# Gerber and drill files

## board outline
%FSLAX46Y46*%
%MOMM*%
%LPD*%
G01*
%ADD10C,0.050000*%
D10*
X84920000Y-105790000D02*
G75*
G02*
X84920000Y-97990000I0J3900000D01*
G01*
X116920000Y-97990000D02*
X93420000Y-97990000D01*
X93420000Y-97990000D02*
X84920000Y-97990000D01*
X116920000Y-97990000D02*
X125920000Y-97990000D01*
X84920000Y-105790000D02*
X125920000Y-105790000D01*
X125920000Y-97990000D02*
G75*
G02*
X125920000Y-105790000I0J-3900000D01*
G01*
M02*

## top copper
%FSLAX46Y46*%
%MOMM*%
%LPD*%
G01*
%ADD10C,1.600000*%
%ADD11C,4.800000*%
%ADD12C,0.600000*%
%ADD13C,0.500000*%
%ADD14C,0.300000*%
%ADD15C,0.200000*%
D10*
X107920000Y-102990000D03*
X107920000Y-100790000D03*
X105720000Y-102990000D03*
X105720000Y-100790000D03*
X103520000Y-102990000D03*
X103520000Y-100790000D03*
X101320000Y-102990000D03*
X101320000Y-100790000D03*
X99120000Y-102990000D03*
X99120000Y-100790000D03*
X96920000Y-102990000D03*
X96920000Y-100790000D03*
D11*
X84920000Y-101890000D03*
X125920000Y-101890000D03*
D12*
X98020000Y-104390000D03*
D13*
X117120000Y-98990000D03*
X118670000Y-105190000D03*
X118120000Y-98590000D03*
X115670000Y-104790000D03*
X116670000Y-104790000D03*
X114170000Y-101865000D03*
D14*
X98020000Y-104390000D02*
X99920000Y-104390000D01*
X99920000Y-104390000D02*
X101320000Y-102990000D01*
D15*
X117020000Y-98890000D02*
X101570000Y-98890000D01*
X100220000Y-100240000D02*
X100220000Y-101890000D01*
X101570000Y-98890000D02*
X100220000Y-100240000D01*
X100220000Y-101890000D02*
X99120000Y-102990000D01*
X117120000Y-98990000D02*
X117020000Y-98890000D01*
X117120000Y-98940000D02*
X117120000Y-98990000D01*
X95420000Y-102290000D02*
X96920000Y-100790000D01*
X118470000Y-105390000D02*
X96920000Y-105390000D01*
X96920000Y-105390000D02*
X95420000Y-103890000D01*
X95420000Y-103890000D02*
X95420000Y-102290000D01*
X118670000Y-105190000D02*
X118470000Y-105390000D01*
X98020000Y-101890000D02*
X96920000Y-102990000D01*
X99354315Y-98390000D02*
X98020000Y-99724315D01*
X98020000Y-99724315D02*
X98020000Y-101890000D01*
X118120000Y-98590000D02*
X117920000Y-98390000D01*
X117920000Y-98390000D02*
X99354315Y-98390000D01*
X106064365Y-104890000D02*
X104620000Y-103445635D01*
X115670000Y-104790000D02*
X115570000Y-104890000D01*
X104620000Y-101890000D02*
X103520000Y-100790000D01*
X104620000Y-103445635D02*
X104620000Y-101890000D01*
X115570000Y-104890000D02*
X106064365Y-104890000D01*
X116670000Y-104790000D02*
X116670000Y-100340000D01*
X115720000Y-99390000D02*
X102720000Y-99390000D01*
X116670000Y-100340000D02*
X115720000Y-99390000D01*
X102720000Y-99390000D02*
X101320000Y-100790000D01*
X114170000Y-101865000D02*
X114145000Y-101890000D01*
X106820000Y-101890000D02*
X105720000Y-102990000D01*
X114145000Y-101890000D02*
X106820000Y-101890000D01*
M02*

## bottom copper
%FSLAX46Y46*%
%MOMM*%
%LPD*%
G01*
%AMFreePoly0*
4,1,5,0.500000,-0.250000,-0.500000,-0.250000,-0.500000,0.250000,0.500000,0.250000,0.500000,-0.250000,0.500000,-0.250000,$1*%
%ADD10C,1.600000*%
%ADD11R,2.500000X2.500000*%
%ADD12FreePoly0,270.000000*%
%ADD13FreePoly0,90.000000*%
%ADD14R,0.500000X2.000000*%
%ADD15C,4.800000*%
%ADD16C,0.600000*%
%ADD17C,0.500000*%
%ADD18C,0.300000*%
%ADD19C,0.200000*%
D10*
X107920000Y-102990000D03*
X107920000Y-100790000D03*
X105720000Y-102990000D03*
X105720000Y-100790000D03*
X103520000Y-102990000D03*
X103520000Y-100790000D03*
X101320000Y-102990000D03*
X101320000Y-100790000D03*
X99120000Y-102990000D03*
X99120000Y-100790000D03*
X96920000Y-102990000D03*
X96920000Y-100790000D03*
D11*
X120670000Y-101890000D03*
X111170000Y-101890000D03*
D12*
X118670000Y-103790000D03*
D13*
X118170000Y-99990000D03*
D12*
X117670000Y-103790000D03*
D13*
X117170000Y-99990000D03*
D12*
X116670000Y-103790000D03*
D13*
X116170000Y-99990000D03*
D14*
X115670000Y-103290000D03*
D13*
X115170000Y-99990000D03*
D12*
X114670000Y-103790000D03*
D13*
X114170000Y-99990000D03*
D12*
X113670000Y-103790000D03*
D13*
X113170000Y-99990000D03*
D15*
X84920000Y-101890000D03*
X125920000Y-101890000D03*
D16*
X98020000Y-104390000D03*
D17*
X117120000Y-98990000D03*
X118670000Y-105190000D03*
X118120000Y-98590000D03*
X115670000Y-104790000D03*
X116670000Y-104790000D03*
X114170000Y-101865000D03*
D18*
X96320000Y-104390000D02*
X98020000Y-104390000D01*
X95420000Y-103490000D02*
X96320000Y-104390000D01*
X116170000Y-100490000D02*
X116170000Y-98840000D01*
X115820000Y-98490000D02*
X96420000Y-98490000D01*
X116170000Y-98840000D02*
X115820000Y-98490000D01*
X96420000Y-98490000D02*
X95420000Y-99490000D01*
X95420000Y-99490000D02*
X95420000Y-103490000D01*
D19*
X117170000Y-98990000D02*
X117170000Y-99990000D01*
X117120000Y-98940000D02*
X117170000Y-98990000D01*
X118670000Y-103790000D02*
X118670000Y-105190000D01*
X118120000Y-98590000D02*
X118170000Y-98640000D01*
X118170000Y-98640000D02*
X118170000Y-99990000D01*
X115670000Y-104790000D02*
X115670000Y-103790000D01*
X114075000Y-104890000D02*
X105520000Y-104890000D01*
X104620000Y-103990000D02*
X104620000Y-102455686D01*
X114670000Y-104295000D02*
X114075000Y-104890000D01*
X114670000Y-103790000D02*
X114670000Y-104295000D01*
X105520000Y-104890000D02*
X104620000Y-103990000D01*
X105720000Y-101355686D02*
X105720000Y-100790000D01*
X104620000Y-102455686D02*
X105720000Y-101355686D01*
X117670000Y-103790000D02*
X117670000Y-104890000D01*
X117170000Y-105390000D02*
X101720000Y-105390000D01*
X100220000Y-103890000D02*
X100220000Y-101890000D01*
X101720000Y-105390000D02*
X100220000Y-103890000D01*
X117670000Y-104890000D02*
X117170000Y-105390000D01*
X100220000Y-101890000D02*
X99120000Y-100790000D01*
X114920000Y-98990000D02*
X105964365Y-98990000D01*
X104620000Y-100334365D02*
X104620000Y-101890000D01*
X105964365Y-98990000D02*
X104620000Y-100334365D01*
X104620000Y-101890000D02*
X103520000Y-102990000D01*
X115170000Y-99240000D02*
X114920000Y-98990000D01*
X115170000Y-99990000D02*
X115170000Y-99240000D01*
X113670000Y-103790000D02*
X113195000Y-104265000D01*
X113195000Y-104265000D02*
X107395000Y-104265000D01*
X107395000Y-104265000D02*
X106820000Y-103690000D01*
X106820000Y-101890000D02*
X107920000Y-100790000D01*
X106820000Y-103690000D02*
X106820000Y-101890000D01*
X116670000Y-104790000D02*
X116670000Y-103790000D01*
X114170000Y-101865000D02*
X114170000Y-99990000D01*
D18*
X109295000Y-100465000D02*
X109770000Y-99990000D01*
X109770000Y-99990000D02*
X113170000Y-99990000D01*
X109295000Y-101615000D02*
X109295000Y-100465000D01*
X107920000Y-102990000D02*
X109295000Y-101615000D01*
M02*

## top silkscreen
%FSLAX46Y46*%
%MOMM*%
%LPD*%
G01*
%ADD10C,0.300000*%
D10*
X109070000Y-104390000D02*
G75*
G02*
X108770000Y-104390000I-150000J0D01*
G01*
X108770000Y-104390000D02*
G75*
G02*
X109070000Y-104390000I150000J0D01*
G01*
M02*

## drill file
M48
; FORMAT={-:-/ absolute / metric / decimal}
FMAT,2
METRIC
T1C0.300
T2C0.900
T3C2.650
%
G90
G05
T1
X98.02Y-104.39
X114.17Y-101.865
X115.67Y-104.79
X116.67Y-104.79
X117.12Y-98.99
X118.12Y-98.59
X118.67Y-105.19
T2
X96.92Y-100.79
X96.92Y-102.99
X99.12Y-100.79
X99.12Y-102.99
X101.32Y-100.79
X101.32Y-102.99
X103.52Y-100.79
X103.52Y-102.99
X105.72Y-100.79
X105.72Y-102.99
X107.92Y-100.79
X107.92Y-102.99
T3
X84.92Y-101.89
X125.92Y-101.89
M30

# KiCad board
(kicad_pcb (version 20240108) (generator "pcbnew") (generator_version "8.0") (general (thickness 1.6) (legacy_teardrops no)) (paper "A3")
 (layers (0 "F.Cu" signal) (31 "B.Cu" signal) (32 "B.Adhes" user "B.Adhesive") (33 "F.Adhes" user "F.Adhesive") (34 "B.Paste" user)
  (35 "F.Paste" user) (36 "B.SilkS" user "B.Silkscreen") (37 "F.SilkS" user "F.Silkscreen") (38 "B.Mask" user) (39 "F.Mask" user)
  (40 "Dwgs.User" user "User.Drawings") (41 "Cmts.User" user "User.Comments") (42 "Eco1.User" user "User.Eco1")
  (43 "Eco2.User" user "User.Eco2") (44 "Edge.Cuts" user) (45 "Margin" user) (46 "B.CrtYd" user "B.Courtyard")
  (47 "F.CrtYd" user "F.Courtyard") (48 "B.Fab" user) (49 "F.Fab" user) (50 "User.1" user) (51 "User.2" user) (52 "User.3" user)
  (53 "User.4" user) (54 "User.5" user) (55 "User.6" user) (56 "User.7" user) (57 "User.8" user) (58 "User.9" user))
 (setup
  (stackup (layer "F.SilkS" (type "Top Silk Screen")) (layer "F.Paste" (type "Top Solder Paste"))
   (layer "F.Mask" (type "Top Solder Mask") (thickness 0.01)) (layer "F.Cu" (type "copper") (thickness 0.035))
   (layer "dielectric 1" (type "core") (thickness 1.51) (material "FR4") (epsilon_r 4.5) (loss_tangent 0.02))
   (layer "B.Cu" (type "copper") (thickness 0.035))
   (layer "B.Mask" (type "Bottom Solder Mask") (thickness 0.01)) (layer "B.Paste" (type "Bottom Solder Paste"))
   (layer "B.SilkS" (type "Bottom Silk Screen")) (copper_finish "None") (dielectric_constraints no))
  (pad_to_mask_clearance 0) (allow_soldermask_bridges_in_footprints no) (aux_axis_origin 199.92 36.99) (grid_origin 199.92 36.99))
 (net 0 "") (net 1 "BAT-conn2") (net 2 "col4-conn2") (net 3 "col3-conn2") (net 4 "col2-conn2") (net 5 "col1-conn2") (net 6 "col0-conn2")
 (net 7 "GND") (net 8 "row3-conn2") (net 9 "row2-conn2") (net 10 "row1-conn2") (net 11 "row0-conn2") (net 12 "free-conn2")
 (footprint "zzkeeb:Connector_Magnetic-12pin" (layer "F.Cu") (at 102.42 101.89 90)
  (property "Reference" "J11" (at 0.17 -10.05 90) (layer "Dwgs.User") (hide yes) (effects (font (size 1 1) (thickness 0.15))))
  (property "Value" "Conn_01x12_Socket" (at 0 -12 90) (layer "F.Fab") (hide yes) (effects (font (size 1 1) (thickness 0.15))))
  (fp_circle (center -2.5 6.5) (end -2.25 6.5) (stroke (width 0.1) (type solid)) (fill solid) (layer "F.SilkS"))
  (pad "1" thru_hole circle (at -1.1 5.5 270) (size 1.6 1.6) (drill 0.9) (layers "*.Cu" "*.Mask") (remove_unused_layers no)
   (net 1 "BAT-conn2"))
  (pad "2" thru_hole circle (at 1.1 5.5 270) (size 1.6 1.6) (drill 0.9) (layers "*.Cu" "*.Mask") (remove_unused_layers no)
   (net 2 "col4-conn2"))
  (pad "3" thru_hole circle (at -1.1 3.3 270) (size 1.6 1.6) (drill 0.9) (layers "*.Cu" "*.Mask") (remove_unused_layers no)
   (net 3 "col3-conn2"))
  (pad "4" thru_hole circle (at 1.1 3.3 270) (size 1.6 1.6) (drill 0.9) (layers "*.Cu" "*.Mask") (remove_unused_layers no)
   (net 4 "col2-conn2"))
  (pad "5" thru_hole circle (at -1.1 1.1 270) (size 1.6 1.6) (drill 0.9) (layers "*.Cu" "*.Mask") (remove_unused_layers no)
   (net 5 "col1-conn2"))
  (pad "6" thru_hole circle (at 1.1 1.1 270) (size 1.6 1.6) (drill 0.9) (layers "*.Cu" "*.Mask") (remove_unused_layers no)
   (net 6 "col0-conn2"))
  (pad "7" thru_hole circle (at -1.1 -1.1 270) (size 1.6 1.6) (drill 0.9) (layers "*.Cu" "*.Mask") (remove_unused_layers no) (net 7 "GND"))
  (pad "8" thru_hole circle (at 1.1 -1.1 270) (size 1.6 1.6) (drill 0.9) (layers "*.Cu" "*.Mask") (remove_unused_layers no)
   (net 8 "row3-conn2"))
  (pad "9" thru_hole circle (at -1.1 -3.3 270) (size 1.6 1.6) (drill 0.9) (layers "*.Cu" "*.Mask") (remove_unused_layers no)
   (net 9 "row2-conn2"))
  (pad "10" thru_hole circle (at 1.1 -3.3 270) (size 1.6 1.6) (drill 0.9) (layers "*.Cu" "*.Mask") (remove_unused_layers no)
   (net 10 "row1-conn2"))
  (pad "11" thru_hole circle (at -1.1 -5.5 270) (size 1.6 1.6) (drill 0.9) (layers "*.Cu" "*.Mask") (remove_unused_layers no)
   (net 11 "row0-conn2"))
  (pad "12" thru_hole circle (at 1.1 -5.5 270) (size 1.6 1.6) (drill 0.9) (layers "*.Cu" "*.Mask") (remove_unused_layers no)
   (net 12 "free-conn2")))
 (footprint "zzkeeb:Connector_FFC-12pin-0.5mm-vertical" (layer "B.Cu") (at 115.92 101.89 180)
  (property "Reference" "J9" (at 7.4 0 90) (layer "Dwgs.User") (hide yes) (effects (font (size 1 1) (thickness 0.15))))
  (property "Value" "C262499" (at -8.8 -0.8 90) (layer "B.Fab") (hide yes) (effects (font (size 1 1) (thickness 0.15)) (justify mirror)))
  (pad "" smd rect (at -4.75 0 90) (size 2.5 2.5) (layers "B.Cu" "B.Paste" "B.Mask"))
  (pad "" smd rect (at 4.75 0 90) (size 2.5 2.5) (layers "B.Cu" "B.Paste" "B.Mask"))
  (pad "1" smd custom (at -2.75 -1.9 270) (size 1 0.5) (layers "B.Cu" "B.Paste" "B.Mask") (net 12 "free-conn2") (thermal_bridge_angle 45)
   (options (clearance outline) (anchor rect)) (primitives))
  (pad "2" smd custom (at -2.25 1.9 90) (size 1 0.5) (layers "B.Cu" "B.Paste" "B.Mask") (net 11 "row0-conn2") (thermal_bridge_angle 45)
   (options (clearance outline) (anchor rect)) (primitives))
  (pad "3" smd custom (at -1.75 -1.9 270) (size 1 0.5) (layers "B.Cu" "B.Paste" "B.Mask") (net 10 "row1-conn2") (thermal_bridge_angle 45)
   (options (clearance outline) (anchor rect)) (primitives))
  (pad "4" smd custom (at -1.25 1.9 90) (size 1 0.5) (layers "B.Cu" "B.Paste" "B.Mask") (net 9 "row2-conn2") (thermal_bridge_angle 45)
   (options (clearance outline) (anchor rect)) (primitives))
  (pad "5" smd custom (at -0.75 -1.9 270) (size 1 0.5) (layers "B.Cu" "B.Paste" "B.Mask") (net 8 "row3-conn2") (thermal_bridge_angle 45)
   (options (clearance outline) (anchor rect)) (primitives))
  (pad "6" smd custom (at -0.25 1.9 90) (size 1 0.5) (layers "B.Cu" "B.Paste" "B.Mask") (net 7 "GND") (thermal_bridge_angle 45)
   (options (clearance outline) (anchor rect)) (primitives))
  (pad "7" smd rect (at 0.25 -1.4 180) (size 0.5 2) (layers "B.Cu" "B.Paste" "B.Mask") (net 6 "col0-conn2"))
  (pad "8" smd custom (at 0.75 1.9 90) (size 1 0.5) (layers "B.Cu" "B.Paste" "B.Mask") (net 5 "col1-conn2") (thermal_bridge_angle 45)
   (options (clearance outline) (anchor rect)) (primitives))
  (pad "9" smd custom (at 1.25 -1.9 270) (size 1 0.5) (layers "B.Cu" "B.Paste" "B.Mask") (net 4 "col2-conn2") (thermal_bridge_angle 45)
   (options (clearance outline) (anchor rect)) (primitives))
  (pad "10" smd custom (at 1.75 1.9 90) (size 1 0.5) (layers "B.Cu" "B.Paste" "B.Mask") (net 3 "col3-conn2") (thermal_bridge_angle 45)
   (options (clearance outline) (anchor rect)) (primitives))
  (pad "11" smd custom (at 2.25 -1.9 270) (size 1 0.5) (layers "B.Cu" "B.Paste" "B.Mask") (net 2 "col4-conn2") (thermal_bridge_angle 45)
   (options (clearance outline) (anchor rect)) (primitives))
  (pad "12" smd custom (at 2.75 1.9 90) (size 1 0.5) (layers "B.Cu" "B.Paste" "B.Mask") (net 1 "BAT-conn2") (thermal_bridge_angle 45)
   (options (clearance outline) (anchor rect)) (primitives)))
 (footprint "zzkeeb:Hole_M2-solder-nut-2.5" (layer "B.Cu") (at 84.92 101.89 -90)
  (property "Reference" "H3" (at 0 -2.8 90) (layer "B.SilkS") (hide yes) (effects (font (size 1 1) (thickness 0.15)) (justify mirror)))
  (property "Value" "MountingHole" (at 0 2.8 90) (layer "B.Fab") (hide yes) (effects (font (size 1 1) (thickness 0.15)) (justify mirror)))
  (pad "" thru_hole circle (at 0 0 270) (size 4.8 4.8) (drill 2.65) (layers "*.Cu" "B.Mask") (remove_unused_layers no)))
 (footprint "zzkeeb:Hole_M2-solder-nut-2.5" (layer "B.Cu") (at 125.92 101.89 -90)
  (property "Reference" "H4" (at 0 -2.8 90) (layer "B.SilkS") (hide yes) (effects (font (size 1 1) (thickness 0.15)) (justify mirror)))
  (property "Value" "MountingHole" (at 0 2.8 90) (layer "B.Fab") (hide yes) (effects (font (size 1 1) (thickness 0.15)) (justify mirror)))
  (pad "" thru_hole circle (at 0 0 270) (size 4.8 4.8) (drill 2.65) (layers "*.Cu" "B.Mask") (remove_unused_layers no)))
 (gr_arc (start 84.92 105.79) (mid 81.02 101.89) (end 84.92 97.99) (stroke (width 0.05) (type default)) (layer "Edge.Cuts"))
 (gr_line (start 116.92 97.99) (end 93.42 97.99) (stroke (width 0.05) (type default)) (layer "Edge.Cuts"))
 (gr_line (start 93.42 97.99) (end 84.92 97.99) (stroke (width 0.05) (type default)) (layer "Edge.Cuts"))
 (gr_line (start 116.92 97.99) (end 125.92 97.99) (stroke (width 0.05) (type default)) (layer "Edge.Cuts"))
 (gr_line (start 84.92 105.79) (end 125.92 105.79) (stroke (width 0.05) (type default)) (layer "Edge.Cuts"))
 (gr_arc (start 125.92 97.99) (mid 129.82 101.89) (end 125.92 105.79) (stroke (width 0.05) (type default)) (layer "Edge.Cuts"))
 (segment (start 98.02 104.39) (end 99.92 104.39) (width 0.3) (layer "F.Cu") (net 7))
 (segment (start 99.92 104.39) (end 101.32 102.99) (width 0.3) (layer "F.Cu") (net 7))
 (via (at 98.02 104.39) (size 0.6) (drill 0.3) (layers "F.Cu" "B.Cu") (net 7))
 (segment (start 96.32 104.39) (end 98.02 104.39) (width 0.3) (layer "B.Cu") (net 7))
 (segment (start 95.42 103.49) (end 96.32 104.39) (width 0.3) (layer "B.Cu") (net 7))
 (segment (start 116.17 100.49) (end 116.17 98.84) (width 0.3) (layer "B.Cu") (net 7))
 (segment (start 115.82 98.49) (end 96.42 98.49) (width 0.3) (layer "B.Cu") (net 7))
 (segment (start 116.17 98.84) (end 115.82 98.49) (width 0.3) (layer "B.Cu") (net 7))
 (segment (start 96.42 98.49) (end 95.42 99.49) (width 0.3) (layer "B.Cu") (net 7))
 (segment (start 95.42 99.49) (end 95.42 103.49) (width 0.3) (layer "B.Cu") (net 7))
 (segment (start 117.02 98.89) (end 101.57 98.89) (width 0.2) (layer "F.Cu") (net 9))
 (segment (start 100.22 100.24) (end 100.22 101.89) (width 0.2) (layer "F.Cu") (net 9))
 (segment (start 101.57 98.89) (end 100.22 100.24) (width 0.2) (layer "F.Cu") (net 9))
 (segment (start 100.22 101.89) (end 99.12 102.99) (width 0.2) (layer "F.Cu") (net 9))
 (segment (start 117.12 98.99) (end 117.02 98.89) (width 0.2) (layer "F.Cu") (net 9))
 (segment (start 117.12 98.94) (end 117.12 98.99) (width 0.2) (layer "F.Cu") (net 9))
 (via (at 117.12 98.99) (size 0.5) (drill 0.3) (layers "F.Cu" "B.Cu") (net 9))
 (segment (start 117.17 98.99) (end 117.17 99.99) (width 0.2) (layer "B.Cu") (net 9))
 (segment (start 117.12 98.94) (end 117.17 98.99) (width 0.2) (layer "B.Cu") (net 9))
 (segment (start 95.42 102.29) (end 96.92 100.79) (width 0.2) (layer "F.Cu") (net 12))
 (segment (start 118.47 105.39) (end 96.92 105.39) (width 0.2) (layer "F.Cu") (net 12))
 (segment (start 96.92 105.39) (end 95.42 103.89) (width 0.2) (layer "F.Cu") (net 12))
 (segment (start 95.42 103.89) (end 95.42 102.29) (width 0.2) (layer "F.Cu") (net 12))
 (segment (start 118.67 105.19) (end 118.47 105.39) (width 0.2) (layer "F.Cu") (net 12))
 (via (at 118.67 105.19) (size 0.5) (drill 0.3) (layers "F.Cu" "B.Cu") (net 12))
 (segment (start 118.67 103.79) (end 118.67 105.19) (width 0.2) (layer "B.Cu") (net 12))
 (segment (start 98.02 101.89) (end 96.92 102.99) (width 0.2) (layer "F.Cu") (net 11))
 (segment (start 99.354315 98.39) (end 98.02 99.724315) (width 0.2) (layer "F.Cu") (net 11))
 (segment (start 98.02 99.724315) (end 98.02 101.89) (width 0.2) (layer "F.Cu") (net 11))
 (segment (start 118.12 98.59) (end 117.92 98.39) (width 0.2) (layer "F.Cu") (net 11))
 (segment (start 117.92 98.39) (end 99.354315 98.39) (width 0.2) (layer "F.Cu") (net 11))
 (via (at 118.12 98.59) (size 0.5) (drill 0.3) (layers "F.Cu" "B.Cu") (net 11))
 (segment (start 118.12 98.59) (end 118.17 98.64) (width 0.2) (layer "B.Cu") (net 11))
 (segment (start 118.17 98.64) (end 118.17 99.99) (width 0.2) (layer "B.Cu") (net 11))
 (segment (start 106.064365 104.89) (end 104.62 103.445635) (width 0.2) (layer "F.Cu") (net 6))
 (segment (start 115.67 104.79) (end 115.57 104.89) (width 0.2) (layer "F.Cu") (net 6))
 (segment (start 104.62 101.89) (end 103.52 100.79) (width 0.2) (layer "F.Cu") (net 6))
 (segment (start 104.62 103.445635) (end 104.62 101.89) (width 0.2) (layer "F.Cu") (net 6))
 (segment (start 115.57 104.89) (end 106.064365 104.89) (width 0.2) (layer "F.Cu") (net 6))
 (via (at 115.67 104.79) (size 0.5) (drill 0.3) (layers "F.Cu" "B.Cu") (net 6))
 (segment (start 115.67 104.79) (end 115.67 103.79) (width 0.2) (layer "B.Cu") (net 6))
 (segment (start 114.075 104.89) (end 105.52 104.89) (width 0.2) (layer "B.Cu") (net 4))
 (segment (start 104.62 103.99) (end 104.62 102.455686) (width 0.2) (layer "B.Cu") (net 4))
 (segment (start 114.67 104.295) (end 114.075 104.89) (width 0.2) (layer "B.Cu") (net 4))
 (segment (start 114.67 103.79) (end 114.67 104.295) (width 0.2) (layer "B.Cu") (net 4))
 (segment (start 105.52 104.89) (end 104.62 103.99) (width 0.2) (layer "B.Cu") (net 4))
 (segment (start 105.72 101.355686) (end 105.72 100.79) (width 0.2) (layer "B.Cu") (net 4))
 (segment (start 104.62 102.455686) (end 105.72 101.355686) (width 0.2) (layer "B.Cu") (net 4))
 (segment (start 117.67 103.79) (end 117.67 104.89) (width 0.2) (layer "B.Cu") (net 10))
 (segment (start 117.17 105.39) (end 101.72 105.39) (width 0.2) (layer "B.Cu") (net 10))
 (segment (start 100.22 103.89) (end 100.22 101.89) (width 0.2) (layer "B.Cu") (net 10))
 (segment (start 101.72 105.39) (end 100.22 103.89) (width 0.2) (layer "B.Cu") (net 10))
 (segment (start 117.67 104.89) (end 117.17 105.39) (width 0.2) (layer "B.Cu") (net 10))
 (segment (start 100.22 101.89) (end 99.12 100.79) (width 0.2) (layer "B.Cu") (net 10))
 (segment (start 114.92 98.99) (end 105.964365 98.99) (width 0.2) (layer "B.Cu") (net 5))
 (segment (start 104.62 100.334365) (end 104.62 101.89) (width 0.2) (layer "B.Cu") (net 5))
 (segment (start 105.964365 98.99) (end 104.62 100.334365) (width 0.2) (layer "B.Cu") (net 5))
 (segment (start 104.62 101.89) (end 103.52 102.99) (width 0.2) (layer "B.Cu") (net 5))
 (segment (start 115.17 99.24) (end 114.92 98.99) (width 0.2) (layer "B.Cu") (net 5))
 (segment (start 115.17 99.99) (end 115.17 99.24) (width 0.2) (layer "B.Cu") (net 5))
 (segment (start 113.67 103.79) (end 113.195 104.265) (width 0.2) (layer "B.Cu") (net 2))
 (segment (start 113.195 104.265) (end 107.395 104.265) (width 0.2) (layer "B.Cu") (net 2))
 (segment (start 107.395 104.265) (end 106.82 103.69) (width 0.2) (layer "B.Cu") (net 2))
 (segment (start 106.82 101.89) (end 107.92 100.79) (width 0.2) (layer "B.Cu") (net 2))
 (segment (start 106.82 103.69) (end 106.82 101.89) (width 0.2) (layer "B.Cu") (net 2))
 (segment (start 116.67 104.79) (end 116.67 100.34) (width 0.2) (layer "F.Cu") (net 8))
 (segment (start 115.72 99.39) (end 102.72 99.39) (width 0.2) (layer "F.Cu") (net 8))
 (segment (start 116.67 100.34) (end 115.72 99.39) (width 0.2) (layer "F.Cu") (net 8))
 (segment (start 102.72 99.39) (end 101.32 100.79) (width 0.2) (layer "F.Cu") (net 8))
 (via (at 116.67 104.79) (size 0.5) (drill 0.3) (layers "F.Cu" "B.Cu") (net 8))
 (segment (start 116.67 104.79) (end 116.67 103.79) (width 0.2) (layer "B.Cu") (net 8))
 (segment (start 114.17 101.865) (end 114.145 101.89) (width 0.2) (layer "F.Cu") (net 3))
 (segment (start 106.82 101.89) (end 105.72 102.99) (width 0.2) (layer "F.Cu") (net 3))
 (segment (start 114.145 101.89) (end 106.82 101.89) (width 0.2) (layer "F.Cu") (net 3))
 (via (at 114.17 101.865) (size 0.5) (drill 0.3) (layers "F.Cu" "B.Cu") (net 3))
 (segment (start 114.17 101.865) (end 114.17 99.99) (width 0.2) (layer "B.Cu") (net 3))
 (segment (start 109.295 100.465) (end 109.77 99.99) (width 0.3) (layer "B.Cu") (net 1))
 (segment (start 109.77 99.99) (end 113.17 99.99) (width 0.3) (layer "B.Cu") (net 1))
 (segment (start 109.295 101.615) (end 109.295 100.465) (width 0.3) (layer "B.Cu") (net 1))
 (segment (start 107.92 102.99) (end 109.295 101.615) (width 0.3) (layer "B.Cu") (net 1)))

